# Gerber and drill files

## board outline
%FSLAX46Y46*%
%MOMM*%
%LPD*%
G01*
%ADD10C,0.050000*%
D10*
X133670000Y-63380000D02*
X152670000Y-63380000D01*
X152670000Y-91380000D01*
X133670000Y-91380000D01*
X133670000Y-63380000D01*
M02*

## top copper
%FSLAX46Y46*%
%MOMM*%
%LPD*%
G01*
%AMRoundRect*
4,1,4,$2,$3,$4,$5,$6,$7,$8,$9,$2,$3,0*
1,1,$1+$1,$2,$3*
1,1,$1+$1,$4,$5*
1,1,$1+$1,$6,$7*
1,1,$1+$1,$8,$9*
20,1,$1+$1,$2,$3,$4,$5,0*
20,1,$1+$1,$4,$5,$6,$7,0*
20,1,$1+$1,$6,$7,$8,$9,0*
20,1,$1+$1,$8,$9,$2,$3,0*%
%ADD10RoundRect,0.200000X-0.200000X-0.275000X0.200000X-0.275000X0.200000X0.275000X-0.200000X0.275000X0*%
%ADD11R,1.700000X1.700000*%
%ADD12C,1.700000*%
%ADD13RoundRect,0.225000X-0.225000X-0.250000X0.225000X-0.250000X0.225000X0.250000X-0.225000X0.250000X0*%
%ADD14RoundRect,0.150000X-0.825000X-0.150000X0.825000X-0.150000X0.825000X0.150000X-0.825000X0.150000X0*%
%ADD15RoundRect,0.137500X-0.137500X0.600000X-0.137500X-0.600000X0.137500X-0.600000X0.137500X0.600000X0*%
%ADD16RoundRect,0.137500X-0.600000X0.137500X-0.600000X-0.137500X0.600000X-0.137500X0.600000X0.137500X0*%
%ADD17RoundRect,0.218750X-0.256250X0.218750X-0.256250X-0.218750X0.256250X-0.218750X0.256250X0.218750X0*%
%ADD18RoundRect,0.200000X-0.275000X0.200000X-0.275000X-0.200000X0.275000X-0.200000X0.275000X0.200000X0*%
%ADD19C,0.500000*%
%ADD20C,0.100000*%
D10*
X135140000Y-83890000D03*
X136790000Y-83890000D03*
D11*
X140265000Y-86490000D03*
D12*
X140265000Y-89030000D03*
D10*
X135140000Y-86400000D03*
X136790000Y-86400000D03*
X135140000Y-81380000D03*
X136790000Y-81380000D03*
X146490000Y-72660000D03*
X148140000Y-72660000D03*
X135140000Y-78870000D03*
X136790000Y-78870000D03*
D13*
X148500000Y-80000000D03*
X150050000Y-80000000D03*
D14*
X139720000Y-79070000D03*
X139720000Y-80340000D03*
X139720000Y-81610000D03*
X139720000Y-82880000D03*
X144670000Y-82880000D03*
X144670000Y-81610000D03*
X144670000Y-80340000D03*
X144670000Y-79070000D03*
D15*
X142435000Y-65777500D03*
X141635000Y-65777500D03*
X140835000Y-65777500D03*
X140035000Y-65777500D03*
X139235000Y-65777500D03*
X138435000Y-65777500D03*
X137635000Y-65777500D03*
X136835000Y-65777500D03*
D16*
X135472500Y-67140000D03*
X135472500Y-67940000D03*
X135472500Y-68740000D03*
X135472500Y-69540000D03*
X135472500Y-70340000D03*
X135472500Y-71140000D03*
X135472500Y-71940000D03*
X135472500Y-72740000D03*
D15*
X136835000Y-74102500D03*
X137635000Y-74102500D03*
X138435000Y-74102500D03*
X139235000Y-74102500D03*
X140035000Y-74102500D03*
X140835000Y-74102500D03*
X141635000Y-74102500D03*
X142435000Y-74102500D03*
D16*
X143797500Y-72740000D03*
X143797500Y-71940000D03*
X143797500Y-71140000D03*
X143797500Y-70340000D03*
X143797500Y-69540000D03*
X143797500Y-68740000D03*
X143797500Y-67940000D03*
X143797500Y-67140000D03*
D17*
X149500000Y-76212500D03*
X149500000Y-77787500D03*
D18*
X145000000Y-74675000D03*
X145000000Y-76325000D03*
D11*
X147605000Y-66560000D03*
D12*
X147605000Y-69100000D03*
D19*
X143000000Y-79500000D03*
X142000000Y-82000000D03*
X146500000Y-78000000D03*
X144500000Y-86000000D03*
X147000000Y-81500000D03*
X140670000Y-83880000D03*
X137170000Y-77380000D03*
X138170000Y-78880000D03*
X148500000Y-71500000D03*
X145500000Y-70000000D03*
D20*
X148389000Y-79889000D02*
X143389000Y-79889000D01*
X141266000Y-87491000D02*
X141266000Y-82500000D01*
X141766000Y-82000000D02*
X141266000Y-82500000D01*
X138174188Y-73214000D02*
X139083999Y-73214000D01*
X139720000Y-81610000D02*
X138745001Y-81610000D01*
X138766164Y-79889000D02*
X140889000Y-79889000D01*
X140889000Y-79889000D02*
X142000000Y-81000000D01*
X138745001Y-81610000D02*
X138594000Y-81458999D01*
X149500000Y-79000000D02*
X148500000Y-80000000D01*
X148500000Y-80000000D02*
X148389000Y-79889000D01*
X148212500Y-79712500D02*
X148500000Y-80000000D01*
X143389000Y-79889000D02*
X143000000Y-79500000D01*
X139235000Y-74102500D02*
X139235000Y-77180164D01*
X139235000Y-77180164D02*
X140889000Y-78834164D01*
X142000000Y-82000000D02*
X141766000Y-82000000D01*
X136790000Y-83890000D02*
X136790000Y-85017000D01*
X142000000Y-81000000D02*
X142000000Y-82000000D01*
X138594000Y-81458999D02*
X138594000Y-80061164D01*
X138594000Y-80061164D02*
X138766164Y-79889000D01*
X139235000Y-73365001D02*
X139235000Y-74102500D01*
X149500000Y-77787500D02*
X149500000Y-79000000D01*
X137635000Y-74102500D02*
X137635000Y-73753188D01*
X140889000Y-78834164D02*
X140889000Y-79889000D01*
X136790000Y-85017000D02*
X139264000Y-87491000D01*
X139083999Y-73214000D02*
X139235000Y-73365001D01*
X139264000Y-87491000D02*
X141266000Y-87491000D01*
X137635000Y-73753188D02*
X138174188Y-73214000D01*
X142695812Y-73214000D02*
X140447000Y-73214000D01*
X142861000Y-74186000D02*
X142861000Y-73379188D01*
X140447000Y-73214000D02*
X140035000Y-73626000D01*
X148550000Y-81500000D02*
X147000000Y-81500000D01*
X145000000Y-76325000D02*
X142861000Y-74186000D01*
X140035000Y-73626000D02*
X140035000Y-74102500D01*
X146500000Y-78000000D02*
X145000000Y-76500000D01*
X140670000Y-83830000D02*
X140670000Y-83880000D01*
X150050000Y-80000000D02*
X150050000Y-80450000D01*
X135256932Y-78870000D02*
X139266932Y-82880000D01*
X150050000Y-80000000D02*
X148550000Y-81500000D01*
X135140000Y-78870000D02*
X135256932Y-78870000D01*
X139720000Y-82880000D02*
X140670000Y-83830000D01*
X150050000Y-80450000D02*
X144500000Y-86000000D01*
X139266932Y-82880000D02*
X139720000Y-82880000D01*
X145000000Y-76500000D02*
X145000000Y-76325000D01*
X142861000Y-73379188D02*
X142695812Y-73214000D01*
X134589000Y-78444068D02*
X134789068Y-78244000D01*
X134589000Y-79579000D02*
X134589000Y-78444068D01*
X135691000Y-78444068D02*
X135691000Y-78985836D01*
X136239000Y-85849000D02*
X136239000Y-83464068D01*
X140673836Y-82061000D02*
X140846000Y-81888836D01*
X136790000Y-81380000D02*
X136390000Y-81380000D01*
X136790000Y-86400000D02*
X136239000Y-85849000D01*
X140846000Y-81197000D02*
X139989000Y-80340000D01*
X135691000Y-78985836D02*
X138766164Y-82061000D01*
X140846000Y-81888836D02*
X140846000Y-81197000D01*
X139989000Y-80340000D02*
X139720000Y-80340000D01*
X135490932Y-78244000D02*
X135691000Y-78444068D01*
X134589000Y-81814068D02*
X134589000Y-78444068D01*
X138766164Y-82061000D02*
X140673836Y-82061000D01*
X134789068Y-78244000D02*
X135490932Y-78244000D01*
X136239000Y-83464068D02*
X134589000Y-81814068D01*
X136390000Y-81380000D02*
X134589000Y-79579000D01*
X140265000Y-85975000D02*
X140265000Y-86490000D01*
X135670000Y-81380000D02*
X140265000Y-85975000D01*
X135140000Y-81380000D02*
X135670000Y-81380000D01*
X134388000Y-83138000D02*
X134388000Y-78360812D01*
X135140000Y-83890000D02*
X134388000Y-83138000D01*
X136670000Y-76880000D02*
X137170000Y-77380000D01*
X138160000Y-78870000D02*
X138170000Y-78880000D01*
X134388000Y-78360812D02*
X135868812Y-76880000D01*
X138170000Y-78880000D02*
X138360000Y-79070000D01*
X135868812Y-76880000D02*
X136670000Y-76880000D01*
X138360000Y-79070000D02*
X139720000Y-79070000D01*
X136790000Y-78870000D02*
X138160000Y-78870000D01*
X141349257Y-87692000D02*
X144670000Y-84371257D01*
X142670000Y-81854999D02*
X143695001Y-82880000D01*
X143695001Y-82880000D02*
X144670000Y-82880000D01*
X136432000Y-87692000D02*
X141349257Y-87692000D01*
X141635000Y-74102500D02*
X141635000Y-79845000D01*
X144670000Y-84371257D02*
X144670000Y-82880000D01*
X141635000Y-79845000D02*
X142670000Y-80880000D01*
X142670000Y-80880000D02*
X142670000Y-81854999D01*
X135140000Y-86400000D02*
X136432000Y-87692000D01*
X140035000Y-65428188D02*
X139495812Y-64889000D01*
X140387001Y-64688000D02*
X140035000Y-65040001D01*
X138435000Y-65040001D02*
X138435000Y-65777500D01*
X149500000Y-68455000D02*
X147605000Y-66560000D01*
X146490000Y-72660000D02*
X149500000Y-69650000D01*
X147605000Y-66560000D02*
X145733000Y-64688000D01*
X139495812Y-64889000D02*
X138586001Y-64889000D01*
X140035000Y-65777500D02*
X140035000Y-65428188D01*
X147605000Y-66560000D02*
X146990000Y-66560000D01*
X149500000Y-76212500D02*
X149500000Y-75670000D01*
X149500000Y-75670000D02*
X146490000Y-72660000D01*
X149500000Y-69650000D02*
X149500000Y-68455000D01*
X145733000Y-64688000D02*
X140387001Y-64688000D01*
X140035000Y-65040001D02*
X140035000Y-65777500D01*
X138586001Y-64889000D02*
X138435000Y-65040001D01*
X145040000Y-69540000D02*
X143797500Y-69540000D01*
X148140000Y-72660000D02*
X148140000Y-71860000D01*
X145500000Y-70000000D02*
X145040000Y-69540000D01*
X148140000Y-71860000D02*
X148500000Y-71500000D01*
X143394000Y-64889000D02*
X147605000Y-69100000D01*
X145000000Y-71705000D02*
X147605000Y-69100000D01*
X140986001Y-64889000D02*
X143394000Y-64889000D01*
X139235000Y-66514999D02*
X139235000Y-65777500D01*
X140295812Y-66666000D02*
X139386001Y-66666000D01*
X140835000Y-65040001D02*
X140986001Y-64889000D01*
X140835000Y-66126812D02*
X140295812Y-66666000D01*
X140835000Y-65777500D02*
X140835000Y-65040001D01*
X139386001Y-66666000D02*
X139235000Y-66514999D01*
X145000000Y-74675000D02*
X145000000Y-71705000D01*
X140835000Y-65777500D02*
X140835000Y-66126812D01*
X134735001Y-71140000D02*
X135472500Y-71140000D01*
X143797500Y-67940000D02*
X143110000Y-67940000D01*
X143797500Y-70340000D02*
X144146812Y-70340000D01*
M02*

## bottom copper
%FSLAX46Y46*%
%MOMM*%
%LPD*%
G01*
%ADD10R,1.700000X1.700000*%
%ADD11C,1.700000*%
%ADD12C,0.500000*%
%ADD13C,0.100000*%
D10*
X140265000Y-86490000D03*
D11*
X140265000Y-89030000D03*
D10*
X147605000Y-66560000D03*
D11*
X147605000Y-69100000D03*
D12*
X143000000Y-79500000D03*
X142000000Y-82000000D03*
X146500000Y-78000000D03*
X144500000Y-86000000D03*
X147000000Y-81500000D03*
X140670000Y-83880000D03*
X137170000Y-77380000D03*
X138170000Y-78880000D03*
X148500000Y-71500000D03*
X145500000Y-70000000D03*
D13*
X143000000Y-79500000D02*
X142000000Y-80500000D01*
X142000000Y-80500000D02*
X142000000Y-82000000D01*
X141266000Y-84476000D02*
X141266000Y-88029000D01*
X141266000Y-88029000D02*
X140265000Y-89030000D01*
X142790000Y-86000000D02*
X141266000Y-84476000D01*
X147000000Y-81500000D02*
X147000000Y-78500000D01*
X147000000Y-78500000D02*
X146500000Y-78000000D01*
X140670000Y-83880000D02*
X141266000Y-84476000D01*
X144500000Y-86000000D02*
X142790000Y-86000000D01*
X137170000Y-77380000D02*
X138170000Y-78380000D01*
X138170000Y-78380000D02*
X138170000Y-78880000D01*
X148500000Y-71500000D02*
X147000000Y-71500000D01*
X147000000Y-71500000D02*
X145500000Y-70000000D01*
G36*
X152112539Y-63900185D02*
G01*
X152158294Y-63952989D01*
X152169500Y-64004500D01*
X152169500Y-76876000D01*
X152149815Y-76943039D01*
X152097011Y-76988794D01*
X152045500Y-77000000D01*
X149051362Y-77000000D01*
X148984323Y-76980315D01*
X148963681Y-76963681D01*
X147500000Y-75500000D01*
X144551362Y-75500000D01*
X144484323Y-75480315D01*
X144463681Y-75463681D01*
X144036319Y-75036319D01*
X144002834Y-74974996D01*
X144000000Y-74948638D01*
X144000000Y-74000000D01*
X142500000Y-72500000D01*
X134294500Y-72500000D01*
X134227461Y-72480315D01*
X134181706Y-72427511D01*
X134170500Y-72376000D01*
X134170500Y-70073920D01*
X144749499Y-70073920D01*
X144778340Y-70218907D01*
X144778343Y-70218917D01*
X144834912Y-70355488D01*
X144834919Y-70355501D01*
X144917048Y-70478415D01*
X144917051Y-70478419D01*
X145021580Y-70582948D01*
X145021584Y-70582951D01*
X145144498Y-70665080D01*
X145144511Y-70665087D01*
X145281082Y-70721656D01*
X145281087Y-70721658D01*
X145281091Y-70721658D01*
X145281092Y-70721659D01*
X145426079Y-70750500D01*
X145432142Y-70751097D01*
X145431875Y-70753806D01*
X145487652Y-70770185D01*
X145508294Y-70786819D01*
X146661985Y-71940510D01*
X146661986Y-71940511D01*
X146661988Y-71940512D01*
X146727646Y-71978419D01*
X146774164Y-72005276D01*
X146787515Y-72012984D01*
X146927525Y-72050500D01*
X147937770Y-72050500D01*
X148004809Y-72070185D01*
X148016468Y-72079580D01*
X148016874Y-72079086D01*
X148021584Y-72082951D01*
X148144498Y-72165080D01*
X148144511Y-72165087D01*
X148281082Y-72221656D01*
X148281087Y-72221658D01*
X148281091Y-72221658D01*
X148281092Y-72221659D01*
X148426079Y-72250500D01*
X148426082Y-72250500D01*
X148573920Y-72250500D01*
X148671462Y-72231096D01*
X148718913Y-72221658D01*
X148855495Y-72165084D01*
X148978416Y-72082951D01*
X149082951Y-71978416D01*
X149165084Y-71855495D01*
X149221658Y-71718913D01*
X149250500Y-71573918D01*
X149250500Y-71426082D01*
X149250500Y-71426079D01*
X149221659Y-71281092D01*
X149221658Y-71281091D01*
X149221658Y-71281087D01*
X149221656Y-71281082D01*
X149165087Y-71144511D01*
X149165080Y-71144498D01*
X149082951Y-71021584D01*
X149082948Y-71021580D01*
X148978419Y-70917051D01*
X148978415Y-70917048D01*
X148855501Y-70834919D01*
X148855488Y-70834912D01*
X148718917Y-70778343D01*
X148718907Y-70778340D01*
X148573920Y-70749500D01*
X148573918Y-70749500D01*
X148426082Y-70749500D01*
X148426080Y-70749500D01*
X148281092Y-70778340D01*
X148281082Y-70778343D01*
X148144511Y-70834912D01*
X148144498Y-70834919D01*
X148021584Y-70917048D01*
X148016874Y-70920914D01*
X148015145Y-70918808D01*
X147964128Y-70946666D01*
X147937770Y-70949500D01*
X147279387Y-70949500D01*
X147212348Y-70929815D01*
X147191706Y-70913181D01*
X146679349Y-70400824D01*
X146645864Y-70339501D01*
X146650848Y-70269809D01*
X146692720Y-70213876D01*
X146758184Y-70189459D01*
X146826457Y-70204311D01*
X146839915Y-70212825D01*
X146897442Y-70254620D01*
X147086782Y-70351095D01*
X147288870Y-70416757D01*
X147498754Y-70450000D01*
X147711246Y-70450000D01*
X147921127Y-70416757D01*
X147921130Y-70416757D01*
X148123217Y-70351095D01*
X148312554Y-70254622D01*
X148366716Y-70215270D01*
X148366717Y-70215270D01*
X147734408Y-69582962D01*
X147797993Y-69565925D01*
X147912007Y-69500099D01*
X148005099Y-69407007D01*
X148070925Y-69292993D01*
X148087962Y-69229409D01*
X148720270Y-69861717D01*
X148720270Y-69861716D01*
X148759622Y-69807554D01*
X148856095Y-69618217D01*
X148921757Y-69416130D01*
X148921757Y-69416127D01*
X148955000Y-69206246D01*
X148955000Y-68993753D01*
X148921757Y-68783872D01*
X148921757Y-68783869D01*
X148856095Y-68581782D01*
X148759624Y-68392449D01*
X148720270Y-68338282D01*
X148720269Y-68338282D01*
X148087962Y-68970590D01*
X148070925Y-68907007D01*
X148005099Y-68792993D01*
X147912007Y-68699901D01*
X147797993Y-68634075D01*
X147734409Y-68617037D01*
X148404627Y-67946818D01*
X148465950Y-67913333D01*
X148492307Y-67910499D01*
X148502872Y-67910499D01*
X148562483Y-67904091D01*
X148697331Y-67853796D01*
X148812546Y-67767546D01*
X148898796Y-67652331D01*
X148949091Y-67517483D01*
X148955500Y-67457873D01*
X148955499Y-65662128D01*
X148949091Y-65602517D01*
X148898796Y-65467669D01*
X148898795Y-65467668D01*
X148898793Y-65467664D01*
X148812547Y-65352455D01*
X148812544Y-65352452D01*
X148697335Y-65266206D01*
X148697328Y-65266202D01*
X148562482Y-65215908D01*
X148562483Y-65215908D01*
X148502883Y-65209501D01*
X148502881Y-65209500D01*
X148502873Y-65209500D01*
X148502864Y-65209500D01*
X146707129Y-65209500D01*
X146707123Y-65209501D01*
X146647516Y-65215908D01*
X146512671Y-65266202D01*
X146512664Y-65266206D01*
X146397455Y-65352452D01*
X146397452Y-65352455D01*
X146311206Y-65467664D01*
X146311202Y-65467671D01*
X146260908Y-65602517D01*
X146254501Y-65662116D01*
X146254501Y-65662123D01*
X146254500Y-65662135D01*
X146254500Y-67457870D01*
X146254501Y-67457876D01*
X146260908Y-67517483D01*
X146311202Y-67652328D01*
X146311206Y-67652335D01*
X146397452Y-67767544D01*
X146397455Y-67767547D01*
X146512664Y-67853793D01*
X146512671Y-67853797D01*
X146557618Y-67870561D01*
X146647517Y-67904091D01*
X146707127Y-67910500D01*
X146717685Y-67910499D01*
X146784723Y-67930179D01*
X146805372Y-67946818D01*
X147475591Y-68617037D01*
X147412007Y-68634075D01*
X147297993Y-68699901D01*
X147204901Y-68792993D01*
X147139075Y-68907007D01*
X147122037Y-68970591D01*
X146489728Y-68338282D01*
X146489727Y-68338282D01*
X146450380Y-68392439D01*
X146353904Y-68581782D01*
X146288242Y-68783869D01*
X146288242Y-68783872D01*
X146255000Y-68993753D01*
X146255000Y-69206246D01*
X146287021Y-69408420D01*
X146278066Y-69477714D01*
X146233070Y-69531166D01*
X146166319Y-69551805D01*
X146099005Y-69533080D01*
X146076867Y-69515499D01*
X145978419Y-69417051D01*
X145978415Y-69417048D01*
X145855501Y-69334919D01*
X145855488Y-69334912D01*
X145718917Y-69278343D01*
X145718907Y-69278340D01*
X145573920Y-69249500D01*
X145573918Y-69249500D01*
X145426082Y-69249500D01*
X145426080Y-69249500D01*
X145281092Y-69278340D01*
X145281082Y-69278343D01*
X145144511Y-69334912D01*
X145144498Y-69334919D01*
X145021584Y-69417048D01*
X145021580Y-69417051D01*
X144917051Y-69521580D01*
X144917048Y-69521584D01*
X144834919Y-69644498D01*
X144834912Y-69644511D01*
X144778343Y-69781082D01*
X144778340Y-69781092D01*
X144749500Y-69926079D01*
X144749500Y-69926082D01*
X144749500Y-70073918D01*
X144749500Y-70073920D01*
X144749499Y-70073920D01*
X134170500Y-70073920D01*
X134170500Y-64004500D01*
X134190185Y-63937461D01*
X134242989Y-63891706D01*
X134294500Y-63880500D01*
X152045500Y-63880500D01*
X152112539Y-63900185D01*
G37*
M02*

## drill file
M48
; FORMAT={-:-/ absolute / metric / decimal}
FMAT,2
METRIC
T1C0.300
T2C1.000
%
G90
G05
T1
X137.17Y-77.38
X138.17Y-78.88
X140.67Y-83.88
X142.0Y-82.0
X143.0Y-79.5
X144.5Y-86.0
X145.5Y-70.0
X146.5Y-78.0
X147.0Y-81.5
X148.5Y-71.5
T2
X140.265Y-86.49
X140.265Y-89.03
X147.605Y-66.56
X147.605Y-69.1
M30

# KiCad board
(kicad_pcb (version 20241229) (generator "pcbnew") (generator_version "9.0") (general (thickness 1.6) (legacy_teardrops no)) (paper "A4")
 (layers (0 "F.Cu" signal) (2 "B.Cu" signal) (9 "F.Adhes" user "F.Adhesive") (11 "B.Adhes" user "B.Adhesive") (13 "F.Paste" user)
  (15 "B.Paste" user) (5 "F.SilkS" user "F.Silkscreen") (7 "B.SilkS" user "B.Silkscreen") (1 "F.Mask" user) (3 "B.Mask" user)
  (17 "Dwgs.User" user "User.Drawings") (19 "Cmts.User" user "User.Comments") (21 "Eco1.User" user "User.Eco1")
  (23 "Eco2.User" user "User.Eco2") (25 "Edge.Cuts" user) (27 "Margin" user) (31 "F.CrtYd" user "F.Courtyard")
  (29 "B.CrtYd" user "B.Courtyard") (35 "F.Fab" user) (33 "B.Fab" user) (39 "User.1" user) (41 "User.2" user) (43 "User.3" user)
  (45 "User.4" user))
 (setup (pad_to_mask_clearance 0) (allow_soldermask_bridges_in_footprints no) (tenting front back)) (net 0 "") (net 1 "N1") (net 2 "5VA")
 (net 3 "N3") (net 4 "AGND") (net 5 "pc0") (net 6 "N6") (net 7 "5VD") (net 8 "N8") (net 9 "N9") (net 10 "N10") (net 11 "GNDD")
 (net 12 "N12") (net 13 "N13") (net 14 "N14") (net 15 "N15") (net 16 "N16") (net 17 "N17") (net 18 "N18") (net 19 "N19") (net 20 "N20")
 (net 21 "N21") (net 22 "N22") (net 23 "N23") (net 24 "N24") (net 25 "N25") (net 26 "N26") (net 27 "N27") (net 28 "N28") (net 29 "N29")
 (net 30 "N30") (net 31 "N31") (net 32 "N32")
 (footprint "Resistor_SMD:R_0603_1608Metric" (layer "F.Cu") (at 135.965 83.89)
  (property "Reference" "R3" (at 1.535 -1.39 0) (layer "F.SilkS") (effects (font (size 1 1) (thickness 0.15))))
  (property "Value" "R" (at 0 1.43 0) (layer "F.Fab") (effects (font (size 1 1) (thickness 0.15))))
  (pad "1" smd roundrect (at -0.825 0) (size 0.8 0.95) (layers "F.Cu" "F.Mask" "F.Paste") (roundrect_rratio 0.25) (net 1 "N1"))
  (pad "2" smd roundrect (at 0.825 0) (size 0.8 0.95) (layers "F.Cu" "F.Mask" "F.Paste") (roundrect_rratio 0.25) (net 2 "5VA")))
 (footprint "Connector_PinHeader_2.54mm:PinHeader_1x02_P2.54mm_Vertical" (layer "F.Cu") (at 140.265 86.49)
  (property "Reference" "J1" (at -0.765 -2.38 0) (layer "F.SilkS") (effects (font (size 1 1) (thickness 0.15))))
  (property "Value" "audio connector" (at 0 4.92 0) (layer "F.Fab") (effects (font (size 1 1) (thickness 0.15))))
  (pad "1" thru_hole rect (at 0 0) (size 1.7 1.7) (drill 1) (layers "*.Cu" "*.Mask") (remove_unused_layers no) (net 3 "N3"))
  (pad "2" thru_hole circle (at 0 2.54) (size 1.7 1.7) (drill 1) (layers "*.Cu" "*.Mask") (remove_unused_layers no) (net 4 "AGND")))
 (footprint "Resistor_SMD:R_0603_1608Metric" (layer "F.Cu") (at 135.965 86.4)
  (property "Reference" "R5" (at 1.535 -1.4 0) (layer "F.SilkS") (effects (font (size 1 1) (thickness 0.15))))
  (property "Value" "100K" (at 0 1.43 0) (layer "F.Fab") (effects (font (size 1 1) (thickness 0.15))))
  (pad "1" smd roundrect (at -0.825 0) (size 0.8 0.95) (layers "F.Cu" "F.Mask" "F.Paste") (roundrect_rratio 0.25) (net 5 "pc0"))
  (pad "2" smd roundrect (at 0.825 0) (size 0.8 0.95) (layers "F.Cu" "F.Mask" "F.Paste") (roundrect_rratio 0.25) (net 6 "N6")))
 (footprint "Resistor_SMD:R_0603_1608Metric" (layer "F.Cu") (at 135.965 81.38)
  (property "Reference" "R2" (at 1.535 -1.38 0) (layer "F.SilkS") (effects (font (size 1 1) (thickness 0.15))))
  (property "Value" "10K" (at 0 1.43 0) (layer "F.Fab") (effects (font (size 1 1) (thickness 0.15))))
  (pad "1" smd roundrect (at -0.825 0) (size 0.8 0.95) (layers "F.Cu" "F.Mask" "F.Paste") (roundrect_rratio 0.25) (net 3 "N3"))
  (pad "2" smd roundrect (at 0.825 0) (size 0.8 0.95) (layers "F.Cu" "F.Mask" "F.Paste") (roundrect_rratio 0.25) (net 6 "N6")))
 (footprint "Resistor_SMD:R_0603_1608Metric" (layer "F.Cu") (at 147.315 72.66)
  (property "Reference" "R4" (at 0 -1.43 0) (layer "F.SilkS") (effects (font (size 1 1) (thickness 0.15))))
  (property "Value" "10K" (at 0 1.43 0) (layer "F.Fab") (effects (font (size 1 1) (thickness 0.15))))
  (pad "1" smd roundrect (at -0.825 0) (size 0.8 0.95) (layers "F.Cu" "F.Mask" "F.Paste") (roundrect_rratio 0.25) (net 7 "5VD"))
  (pad "2" smd roundrect (at 0.825 0) (size 0.8 0.95) (layers "F.Cu" "F.Mask" "F.Paste") (roundrect_rratio 0.25) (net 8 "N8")))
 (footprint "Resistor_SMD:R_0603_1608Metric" (layer "F.Cu") (at 135.965 78.87)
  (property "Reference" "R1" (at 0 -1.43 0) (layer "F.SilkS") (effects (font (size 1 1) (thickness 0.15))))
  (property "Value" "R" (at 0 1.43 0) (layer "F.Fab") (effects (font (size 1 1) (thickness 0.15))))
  (pad "1" smd roundrect (at -0.825 0) (size 0.8 0.95) (layers "F.Cu" "F.Mask" "F.Paste") (roundrect_rratio 0.25) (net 4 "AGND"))
  (pad "2" smd roundrect (at 0.825 0) (size 0.8 0.95) (layers "F.Cu" "F.Mask" "F.Paste") (roundrect_rratio 0.25) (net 1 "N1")))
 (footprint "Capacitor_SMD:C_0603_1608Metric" (layer "F.Cu") (at 149.275 80)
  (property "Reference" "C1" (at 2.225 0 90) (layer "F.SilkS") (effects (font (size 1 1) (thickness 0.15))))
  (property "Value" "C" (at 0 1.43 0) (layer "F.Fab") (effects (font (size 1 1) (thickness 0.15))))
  (pad "1" smd roundrect (at -0.775 0) (size 0.9 0.95) (layers "F.Cu" "F.Mask" "F.Paste") (roundrect_rratio 0.25) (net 2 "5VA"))
  (pad "2" smd roundrect (at 0.775 0) (size 0.9 0.95) (layers "F.Cu" "F.Mask" "F.Paste") (roundrect_rratio 0.25) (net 4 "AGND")))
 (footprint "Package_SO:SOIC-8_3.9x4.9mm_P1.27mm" (layer "F.Cu") (at 142.195 80.975)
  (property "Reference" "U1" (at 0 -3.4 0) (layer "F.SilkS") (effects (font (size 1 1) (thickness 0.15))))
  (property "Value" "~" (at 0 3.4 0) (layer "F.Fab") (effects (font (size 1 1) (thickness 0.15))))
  (pad "1" smd roundrect (at -2.475 -1.905) (size 1.95 0.6) (layers "F.Cu" "F.Mask" "F.Paste") (roundrect_rratio 0.25) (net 1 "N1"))
  (pad "2" smd roundrect (at -2.475 -0.635) (size 1.95 0.6) (layers "F.Cu" "F.Mask" "F.Paste") (roundrect_rratio 0.25) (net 6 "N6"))
  (pad "3" smd roundrect (at -2.475 0.635) (size 1.95 0.6) (layers "F.Cu" "F.Mask" "F.Paste") (roundrect_rratio 0.25) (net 2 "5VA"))
  (pad "4" smd roundrect (at -2.475 1.905) (size 1.95 0.6) (layers "F.Cu" "F.Mask" "F.Paste") (roundrect_rratio 0.25) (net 4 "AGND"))
  (pad "5" smd roundrect (at 2.475 1.905) (size 1.95 0.6) (layers "F.Cu" "F.Mask" "F.Paste") (roundrect_rratio 0.25) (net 5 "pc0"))
  (pad "6" smd roundrect (at 2.475 0.635) (size 1.95 0.6) (layers "F.Cu" "F.Mask" "F.Paste") (roundrect_rratio 0.25))
  (pad "7" smd roundrect (at 2.475 -0.635) (size 1.95 0.6) (layers "F.Cu" "F.Mask" "F.Paste") (roundrect_rratio 0.25))
  (pad "8" smd roundrect (at 2.475 -1.905) (size 1.95 0.6) (layers "F.Cu" "F.Mask" "F.Paste") (roundrect_rratio 0.25)))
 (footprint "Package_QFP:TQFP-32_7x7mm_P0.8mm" (layer "F.Cu") (at 139.635 69.94 -90)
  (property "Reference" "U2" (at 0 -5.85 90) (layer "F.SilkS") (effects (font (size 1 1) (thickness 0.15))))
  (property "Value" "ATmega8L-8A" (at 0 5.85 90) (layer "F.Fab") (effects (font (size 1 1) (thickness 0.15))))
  (pad "1" smd roundrect (at -4.1625 -2.8 270) (size 1.475 0.55) (layers "F.Cu" "F.Mask" "F.Paste") (roundrect_rratio 0.25) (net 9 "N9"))
  (pad "2" smd roundrect (at -4.1625 -2 270) (size 1.475 0.55) (layers "F.Cu" "F.Mask" "F.Paste") (roundrect_rratio 0.25) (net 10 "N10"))
  (pad "3" smd roundrect (at -4.1625 -1.2 270) (size 1.475 0.55) (layers "F.Cu" "F.Mask" "F.Paste") (roundrect_rratio 0.25) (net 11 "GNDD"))
  (pad "4" smd roundrect (at -4.1625 -0.4 270) (size 1.475 0.55) (layers "F.Cu" "F.Mask" "F.Paste") (roundrect_rratio 0.25) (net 7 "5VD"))
  (pad "5" smd roundrect (at -4.1625 0.4 270) (size 1.475 0.55) (layers "F.Cu" "F.Mask" "F.Paste") (roundrect_rratio 0.25) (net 11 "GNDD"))
  (pad "6" smd roundrect (at -4.1625 1.2 270) (size 1.475 0.55) (layers "F.Cu" "F.Mask" "F.Paste") (roundrect_rratio 0.25) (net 7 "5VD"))
  (pad "7" smd roundrect (at -4.1625 2 270) (size 1.475 0.55) (layers "F.Cu" "F.Mask" "F.Paste") (roundrect_rratio 0.25) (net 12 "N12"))
  (pad "8" smd roundrect (at -4.1625 2.8 270) (size 1.475 0.55) (layers "F.Cu" "F.Mask" "F.Paste") (roundrect_rratio 0.25) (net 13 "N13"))
  (pad "9" smd roundrect (at -2.8 4.1625 270) (size 0.55 1.475) (layers "F.Cu" "F.Mask" "F.Paste") (roundrect_rratio 0.25) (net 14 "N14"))
  (pad "10" smd roundrect (at -2 4.1625 270) (size 0.55 1.475) (layers "F.Cu" "F.Mask" "F.Paste") (roundrect_rratio 0.25) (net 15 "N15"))
  (pad "11" smd roundrect (at -1.2 4.1625 270) (size 0.55 1.475) (layers "F.Cu" "F.Mask" "F.Paste") (roundrect_rratio 0.25) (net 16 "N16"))
  (pad "12" smd roundrect (at -0.4 4.1625 270) (size 0.55 1.475) (layers "F.Cu" "F.Mask" "F.Paste") (roundrect_rratio 0.25) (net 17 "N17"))
  (pad "13" smd roundrect (at 0.4 4.1625 270) (size 0.55 1.475) (layers "F.Cu" "F.Mask" "F.Paste") (roundrect_rratio 0.25) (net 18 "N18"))
  (pad "14" smd roundrect (at 1.2 4.1625 270) (size 0.55 1.475) (layers "F.Cu" "F.Mask" "F.Paste") (roundrect_rratio 0.25) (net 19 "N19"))
  (pad "15" smd roundrect (at 2 4.1625 270) (size 0.55 1.475) (layers "F.Cu" "F.Mask" "F.Paste") (roundrect_rratio 0.25) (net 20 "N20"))
  (pad "16" smd roundrect (at 2.8 4.1625 270) (size 0.55 1.475) (layers "F.Cu" "F.Mask" "F.Paste") (roundrect_rratio 0.25) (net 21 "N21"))
  (pad "17" smd roundrect (at 4.1625 2.8 270) (size 1.475 0.55) (layers "F.Cu" "F.Mask" "F.Paste") (roundrect_rratio 0.25) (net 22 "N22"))
  (pad "18" smd roundrect (at 4.1625 2 270) (size 1.475 0.55) (layers "F.Cu" "F.Mask" "F.Paste") (roundrect_rratio 0.25) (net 2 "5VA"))
  (pad "19" smd roundrect (at 4.1625 1.2 270) (size 1.475 0.55) (layers "F.Cu" "F.Mask" "F.Paste") (roundrect_rratio 0.25) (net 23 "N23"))
  (pad "20" smd roundrect (at 4.1625 0.4 270) (size 1.475 0.55) (layers "F.Cu" "F.Mask" "F.Paste") (roundrect_rratio 0.25) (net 2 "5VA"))
  (pad "21" smd roundrect (at 4.1625 -0.4 270) (size 1.475 0.55) (layers "F.Cu" "F.Mask" "F.Paste") (roundrect_rratio 0.25) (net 4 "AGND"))
  (pad "22" smd roundrect (at 4.1625 -1.2 270) (size 1.475 0.55) (layers "F.Cu" "F.Mask" "F.Paste") (roundrect_rratio 0.25) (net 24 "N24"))
  (pad "23" smd roundrect (at 4.1625 -2 270) (size 1.475 0.55) (layers "F.Cu" "F.Mask" "F.Paste") (roundrect_rratio 0.25) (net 5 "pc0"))
  (pad "24" smd roundrect (at 4.1625 -2.8 270) (size 1.475 0.55) (layers "F.Cu" "F.Mask" "F.Paste") (roundrect_rratio 0.25) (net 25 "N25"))
  (pad "25" smd roundrect (at 2.8 -4.1625 270) (size 0.55 1.475) (layers "F.Cu" "F.Mask" "F.Paste") (roundrect_rratio 0.25) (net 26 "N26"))
  (pad "26" smd roundrect (at 2 -4.1625 270) (size 0.55 1.475) (layers "F.Cu" "F.Mask" "F.Paste") (roundrect_rratio 0.25) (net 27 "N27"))
  (pad "27" smd roundrect (at 1.2 -4.1625 270) (size 0.55 1.475) (layers "F.Cu" "F.Mask" "F.Paste") (roundrect_rratio 0.25) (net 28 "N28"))
  (pad "28" smd roundrect (at 0.4 -4.1625 270) (size 0.55 1.475) (layers "F.Cu" "F.Mask" "F.Paste") (roundrect_rratio 0.25) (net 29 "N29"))
  (pad "29" smd roundrect (at -0.4 -4.1625 270) (size 0.55 1.475) (layers "F.Cu" "F.Mask" "F.Paste") (roundrect_rratio 0.25) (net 8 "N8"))
  (pad "30" smd roundrect (at -1.2 -4.1625 270) (size 0.55 1.475) (layers "F.Cu" "F.Mask" "F.Paste") (roundrect_rratio 0.25) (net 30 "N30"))
  (pad "31" smd roundrect (at -2 -4.1625 270) (size 0.55 1.475) (layers "F.Cu" "F.Mask" "F.Paste") (roundrect_rratio 0.25) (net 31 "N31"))
  (pad "32" smd roundrect (at -2.8 -4.1625 270) (size 0.55 1.475) (layers "F.Cu" "F.Mask" "F.Paste") (roundrect_rratio 0.25) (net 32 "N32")))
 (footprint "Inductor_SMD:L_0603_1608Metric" (layer "F.Cu") (at 149.5 77 -90)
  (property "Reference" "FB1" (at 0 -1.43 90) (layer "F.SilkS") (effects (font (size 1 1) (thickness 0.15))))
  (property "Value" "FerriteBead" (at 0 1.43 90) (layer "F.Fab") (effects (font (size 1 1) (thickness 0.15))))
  (pad "1" smd roundrect (at -0.7875 0 270) (size 0.875 0.95) (layers "F.Cu" "F.Mask" "F.Paste") (roundrect_rratio 0.25) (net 7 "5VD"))
  (pad "2" smd roundrect (at 0.7875 0 270) (size 0.875 0.95) (layers "F.Cu" "F.Mask" "F.Paste") (roundrect_rratio 0.25) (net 2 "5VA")))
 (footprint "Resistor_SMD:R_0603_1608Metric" (layer "F.Cu") (at 145 75.5 -90)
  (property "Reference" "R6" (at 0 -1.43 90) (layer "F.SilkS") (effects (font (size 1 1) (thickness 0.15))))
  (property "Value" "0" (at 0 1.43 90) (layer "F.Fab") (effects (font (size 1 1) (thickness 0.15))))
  (pad "1" smd roundrect (at -0.825 0 270) (size 0.8 0.95) (layers "F.Cu" "F.Mask" "F.Paste") (roundrect_rratio 0.25) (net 11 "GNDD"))
  (pad "2" smd roundrect (at 0.825 0 270) (size 0.8 0.95) (layers "F.Cu" "F.Mask" "F.Paste") (roundrect_rratio 0.25) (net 4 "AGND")))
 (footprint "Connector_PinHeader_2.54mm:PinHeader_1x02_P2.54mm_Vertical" (layer "F.Cu") (at 147.605 66.56)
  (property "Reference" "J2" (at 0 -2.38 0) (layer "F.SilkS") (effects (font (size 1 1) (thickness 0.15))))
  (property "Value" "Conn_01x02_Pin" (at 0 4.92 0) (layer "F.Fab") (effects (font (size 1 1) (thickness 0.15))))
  (pad "1" thru_hole rect (at 0 0) (size 1.7 1.7) (drill 1) (layers "*.Cu" "*.Mask") (remove_unused_layers no) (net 7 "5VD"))
  (pad "2" thru_hole circle (at 0 2.54) (size 1.7 1.7) (drill 1) (layers "*.Cu" "*.Mask") (remove_unused_layers no) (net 11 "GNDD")))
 (gr_rect (start 133.67 63.38) (end 152.67 91.38) (stroke (width 0.05) (type default)) (fill no) (layer "Edge.Cuts"))
 (segment (start 148.389 79.889) (end 143.389 79.889) (width 0.1) (layer "F.Cu") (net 2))
 (segment (start 141.266 87.491) (end 141.266 82.5) (width 0.1) (layer "F.Cu") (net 2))
 (segment (start 141.766 82) (end 141.266 82.5) (width 0.1) (layer "F.Cu") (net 2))
 (segment (start 138.174188 73.214) (end 139.083999 73.214) (width 0.1) (layer "F.Cu") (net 2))
 (segment (start 139.72 81.61) (end 138.745001 81.61) (width 0.1) (layer "F.Cu") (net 2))
 (segment (start 138.766164 79.889) (end 140.889 79.889) (width 0.1) (layer "F.Cu") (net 2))
 (segment (start 140.889 79.889) (end 142 81) (width 0.1) (layer "F.Cu") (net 2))
 (segment (start 138.745001 81.61) (end 138.594 81.458999) (width 0.1) (layer "F.Cu") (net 2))
 (segment (start 149.5 79) (end 148.5 80) (width 0.1) (layer "F.Cu") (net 2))
 (segment (start 148.5 80) (end 148.389 79.889) (width 0.1) (layer "F.Cu") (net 2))
 (segment (start 148.2125 79.7125) (end 148.5 80) (width 0.1) (layer "F.Cu") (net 2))
 (segment (start 143.389 79.889) (end 143 79.5) (width 0.1) (layer "F.Cu") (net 2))
 (segment (start 139.235 74.1025) (end 139.235 77.180164) (width 0.1) (layer "F.Cu") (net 2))
 (segment (start 139.235 77.180164) (end 140.889 78.834164) (width 0.1) (layer "F.Cu") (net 2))
 (segment (start 142 82) (end 141.766 82) (width 0.1) (layer "F.Cu") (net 2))
 (segment (start 136.79 83.89) (end 136.79 85.017) (width 0.1) (layer "F.Cu") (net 2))
 (segment (start 142 81) (end 142 82) (width 0.1) (layer "F.Cu") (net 2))
 (segment (start 138.594 81.458999) (end 138.594 80.061164) (width 0.1) (layer "F.Cu") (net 2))
 (segment (start 138.594 80.061164) (end 138.766164 79.889) (width 0.1) (layer "F.Cu") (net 2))
 (segment (start 139.235 73.365001) (end 139.235 74.1025) (width 0.1) (layer "F.Cu") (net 2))
 (segment (start 149.5 77.7875) (end 149.5 79) (width 0.1) (layer "F.Cu") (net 2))
 (segment (start 137.635 74.1025) (end 137.635 73.753188) (width 0.1) (layer "F.Cu") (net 2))
 (segment (start 140.889 78.834164) (end 140.889 79.889) (width 0.1) (layer "F.Cu") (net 2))
 (segment (start 136.79 85.017) (end 139.264 87.491) (width 0.1) (layer "F.Cu") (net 2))
 (segment (start 139.083999 73.214) (end 139.235 73.365001) (width 0.1) (layer "F.Cu") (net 2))
 (segment (start 139.264 87.491) (end 141.266 87.491) (width 0.1) (layer "F.Cu") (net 2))
 (segment (start 137.635 73.753188) (end 138.174188 73.214) (width 0.1) (layer "F.Cu") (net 2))
 (via (at 143 79.5) (size 0.5) (drill 0.3) (layers "F.Cu" "B.Cu") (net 2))
 (via (at 142 82) (size 0.5) (drill 0.3) (layers "F.Cu" "B.Cu") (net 2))
 (segment (start 143 79.5) (end 142 80.5) (width 0.1) (layer "B.Cu") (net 2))
 (segment (start 142 80.5) (end 142 82) (width 0.1) (layer "B.Cu") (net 2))
 (segment (start 142.695812 73.214) (end 140.447 73.214) (width 0.1) (layer "F.Cu") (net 4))
 (segment (start 142.861 74.186) (end 142.861 73.379188) (width 0.1) (layer "F.Cu") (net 4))
 (segment (start 140.447 73.214) (end 140.035 73.626) (width 0.1) (layer "F.Cu") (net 4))
 (segment (start 148.55 81.5) (end 147 81.5) (width 0.1) (layer "F.Cu") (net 4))
 (segment (start 145 76.325) (end 142.861 74.186) (width 0.1) (layer "F.Cu") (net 4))
 (segment (start 140.035 73.626) (end 140.035 74.1025) (width 0.1) (layer "F.Cu") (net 4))
 (segment (start 146.5 78) (end 145 76.5) (width 0.1) (layer "F.Cu") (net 4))
 (segment (start 140.67 83.83) (end 140.67 83.88) (width 0.1) (layer "F.Cu") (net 4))
 (segment (start 150.05 80) (end 150.05 80.45) (width 0.1) (layer "F.Cu") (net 4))
 (segment (start 135.256932 78.87) (end 139.266932 82.88) (width 0.1) (layer "F.Cu") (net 4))
 (segment (start 150.05 80) (end 148.55 81.5) (width 0.1) (layer "F.Cu") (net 4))
 (segment (start 135.14 78.87) (end 135.256932 78.87) (width 0.1) (layer "F.Cu") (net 4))
 (segment (start 139.72 82.88) (end 140.67 83.83) (width 0.1) (layer "F.Cu") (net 4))
 (segment (start 150.05 80.45) (end 144.5 86) (width 0.1) (layer "F.Cu") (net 4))
 (segment (start 139.266932 82.88) (end 139.72 82.88) (width 0.1) (layer "F.Cu") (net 4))
 (segment (start 145 76.5) (end 145 76.325) (width 0.1) (layer "F.Cu") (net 4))
 (segment (start 142.861 73.379188) (end 142.695812 73.214) (width 0.1) (layer "F.Cu") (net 4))
 (via (at 146.5 78) (size 0.5) (drill 0.3) (layers "F.Cu" "B.Cu") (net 4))
 (via (at 144.5 86) (size 0.5) (drill 0.3) (layers "F.Cu" "B.Cu") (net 4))
 (via (at 147 81.5) (size 0.5) (drill 0.3) (layers "F.Cu" "B.Cu") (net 4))
 (via (at 140.67 83.88) (size 0.5) (drill 0.3) (layers "F.Cu" "B.Cu") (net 4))
 (segment (start 141.266 84.476) (end 141.266 88.029) (width 0.1) (layer "B.Cu") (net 4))
 (segment (start 141.266 88.029) (end 140.265 89.03) (width 0.1) (layer "B.Cu") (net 4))
 (segment (start 142.79 86) (end 141.266 84.476) (width 0.1) (layer "B.Cu") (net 4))
 (segment (start 147 81.5) (end 147 78.5) (width 0.1) (layer "B.Cu") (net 4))
 (segment (start 147 78.5) (end 146.5 78) (width 0.1) (layer "B.Cu") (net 4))
 (segment (start 140.67 83.88) (end 141.266 84.476) (width 0.1) (layer "B.Cu") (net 4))
 (segment (start 144.5 86) (end 142.79 86) (width 0.1) (layer "B.Cu") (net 4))
 (segment (start 134.589 78.444068) (end 134.789068 78.244) (width 0.1) (layer "F.Cu") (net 6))
 (segment (start 134.589 79.579) (end 134.589 78.444068) (width 0.1) (layer "F.Cu") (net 6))
 (segment (start 135.691 78.444068) (end 135.691 78.985836) (width 0.1) (layer "F.Cu") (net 6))
 (segment (start 136.239 85.849) (end 136.239 83.464068) (width 0.1) (layer "F.Cu") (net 6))
 (segment (start 140.673836 82.061) (end 140.846 81.888836) (width 0.1) (layer "F.Cu") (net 6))
 (segment (start 136.79 81.38) (end 136.39 81.38) (width 0.1) (layer "F.Cu") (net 6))
 (segment (start 136.79 86.4) (end 136.239 85.849) (width 0.1) (layer "F.Cu") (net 6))
 (segment (start 140.846 81.197) (end 139.989 80.34) (width 0.1) (layer "F.Cu") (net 6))
 (segment (start 135.691 78.985836) (end 138.766164 82.061) (width 0.1) (layer "F.Cu") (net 6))
 (segment (start 140.846 81.888836) (end 140.846 81.197) (width 0.1) (layer "F.Cu") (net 6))
 (segment (start 139.989 80.34) (end 139.72 80.34) (width 0.1) (layer "F.Cu") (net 6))
 (segment (start 135.490932 78.244) (end 135.691 78.444068) (width 0.1) (layer "F.Cu") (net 6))
 (segment (start 134.589 81.814068) (end 134.589 78.444068) (width 0.1) (layer "F.Cu") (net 6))
 (segment (start 138.766164 82.061) (end 140.673836 82.061) (width 0.1) (layer "F.Cu") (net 6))
 (segment (start 134.789068 78.244) (end 135.490932 78.244) (width 0.1) (layer "F.Cu") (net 6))
 (segment (start 136.239 83.464068) (end 134.589 81.814068) (width 0.1) (layer "F.Cu") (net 6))
 (segment (start 136.39 81.38) (end 134.589 79.579) (width 0.1) (layer "F.Cu") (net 6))
 (segment (start 140.265 85.975) (end 140.265 86.49) (width 0.1) (layer "F.Cu") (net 3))
 (segment (start 135.67 81.38) (end 140.265 85.975) (width 0.1) (layer "F.Cu") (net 3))
 (segment (start 135.14 81.38) (end 135.67 81.38) (width 0.1) (layer "F.Cu") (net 3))
 (segment (start 134.388 83.138) (end 134.388 78.360812) (width 0.1) (layer "F.Cu") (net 1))
 (segment (start 135.14 83.89) (end 134.388 83.138) (width 0.1) (layer "F.Cu") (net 1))
 (segment (start 136.67 76.88) (end 137.17 77.38) (width 0.1) (layer "F.Cu") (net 1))
 (segment (start 138.16 78.87) (end 138.17 78.88) (width 0.1) (layer "F.Cu") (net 1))
 (segment (start 134.388 78.360812) (end 135.868812 76.88) (width 0.1) (layer "F.Cu") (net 1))
 (segment (start 138.17 78.88) (end 138.36 79.07) (width 0.1) (layer "F.Cu") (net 1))
 (segment (start 135.868812 76.88) (end 136.67 76.88) (width 0.1) (layer "F.Cu") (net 1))
 (segment (start 138.36 79.07) (end 139.72 79.07) (width 0.1) (layer "F.Cu") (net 1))
 (segment (start 136.79 78.87) (end 138.16 78.87) (width 0.1) (layer "F.Cu") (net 1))
 (via (at 137.17 77.38) (size 0.5) (drill 0.3) (layers "F.Cu" "B.Cu") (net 1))
 (via (at 138.17 78.88) (size 0.5) (drill 0.3) (layers "F.Cu" "B.Cu") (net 1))
 (segment (start 137.17 77.38) (end 138.17 78.38) (width 0.1) (layer "B.Cu") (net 1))
 (segment (start 138.17 78.38) (end 138.17 78.88) (width 0.1) (layer "B.Cu") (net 1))
 (segment (start 141.349257 87.692) (end 144.67 84.371257) (width 0.1) (layer "F.Cu") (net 5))
 (segment (start 142.67 81.854999) (end 143.695001 82.88) (width 0.1) (layer "F.Cu") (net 5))
 (segment (start 143.695001 82.88) (end 144.67 82.88) (width 0.1) (layer "F.Cu") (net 5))
 (segment (start 136.432 87.692) (end 141.349257 87.692) (width 0.1) (layer "F.Cu") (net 5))
 (segment (start 141.635 74.1025) (end 141.635 79.845) (width 0.1) (layer "F.Cu") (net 5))
 (segment (start 144.67 84.371257) (end 144.67 82.88) (width 0.1) (layer "F.Cu") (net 5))
 (segment (start 141.635 79.845) (end 142.67 80.88) (width 0.1) (layer "F.Cu") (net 5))
 (segment (start 142.67 80.88) (end 142.67 81.854999) (width 0.1) (layer "F.Cu") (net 5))
 (segment (start 135.14 86.4) (end 136.432 87.692) (width 0.1) (layer "F.Cu") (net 5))
 (segment (start 140.035 65.428188) (end 139.495812 64.889) (width 0.1) (layer "F.Cu") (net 7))
 (segment (start 140.387001 64.688) (end 140.035 65.040001) (width 0.1) (layer "F.Cu") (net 7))
 (segment (start 138.435 65.040001) (end 138.435 65.7775) (width 0.1) (layer "F.Cu") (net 7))
 (segment (start 149.5 68.455) (end 147.605 66.56) (width 0.1) (layer "F.Cu") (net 7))
 (segment (start 146.49 72.66) (end 149.5 69.65) (width 0.1) (layer "F.Cu") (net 7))
 (segment (start 147.605 66.56) (end 145.733 64.688) (width 0.1) (layer "F.Cu") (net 7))
 (segment (start 139.495812 64.889) (end 138.586001 64.889) (width 0.1) (layer "F.Cu") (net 7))
 (segment (start 140.035 65.7775) (end 140.035 65.428188) (width 0.1) (layer "F.Cu") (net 7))
 (segment (start 147.605 66.56) (end 146.99 66.56) (width 0.1) (layer "F.Cu") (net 7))
 (segment (start 149.5 76.2125) (end 149.5 75.67) (width 0.1) (layer "F.Cu") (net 7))
 (segment (start 149.5 75.67) (end 146.49 72.66) (width 0.1) (layer "F.Cu") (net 7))
 (segment (start 149.5 69.65) (end 149.5 68.455) (width 0.1) (layer "F.Cu") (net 7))
 (segment (start 145.733 64.688) (end 140.387001 64.688) (width 0.1) (layer "F.Cu") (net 7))
 (segment (start 140.035 65.040001) (end 140.035 65.7775) (width 0.1) (layer "F.Cu") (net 7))
 (segment (start 138.586001 64.889) (end 138.435 65.040001) (width 0.1) (layer "F.Cu") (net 7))
 (segment (start 145.04 69.54) (end 143.7975 69.54) (width 0.1) (layer "F.Cu") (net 8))
 (segment (start 148.14 72.66) (end 148.14 71.86) (width 0.1) (layer "F.Cu") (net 8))
 (segment (start 145.5 70) (end 145.04 69.54) (width 0.1) (layer "F.Cu") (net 8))
 (segment (start 148.14 71.86) (end 148.5 71.5) (width 0.1) (layer "F.Cu") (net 8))
 (via (at 148.5 71.5) (size 0.5) (drill 0.3) (layers "F.Cu" "B.Cu") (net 8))
 (via (at 145.5 70) (size 0.5) (drill 0.3) (layers "F.Cu" "B.Cu") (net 8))
 (segment (start 148.5 71.5) (end 147 71.5) (width 0.1) (layer "B.Cu") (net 8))
 (segment (start 147 71.5) (end 145.5 70) (width 0.1) (layer "B.Cu") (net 8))
 (segment (start 143.394 64.889) (end 147.605 69.1) (width 0.1) (layer "F.Cu") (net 11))
 (segment (start 145 71.705) (end 147.605 69.1) (width 0.1) (layer "F.Cu") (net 11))
 (segment (start 140.986001 64.889) (end 143.394 64.889) (width 0.1) (layer "F.Cu") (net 11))
 (segment (start 139.235 66.514999) (end 139.235 65.7775) (width 0.1) (layer "F.Cu") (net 11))
 (segment (start 140.295812 66.666) (end 139.386001 66.666) (width 0.1) (layer "F.Cu") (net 11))
 (segment (start 140.835 65.040001) (end 140.986001 64.889) (width 0.1) (layer "F.Cu") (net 11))
 (segment (start 140.835 66.126812) (end 140.295812 66.666) (width 0.1) (layer "F.Cu") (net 11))
 (segment (start 140.835 65.7775) (end 140.835 65.040001) (width 0.1) (layer "F.Cu") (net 11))
 (segment (start 139.386001 66.666) (end 139.235 66.514999) (width 0.1) (layer "F.Cu") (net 11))
 (segment (start 145 74.675) (end 145 71.705) (width 0.1) (layer "F.Cu") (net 11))
 (segment (start 140.835 65.7775) (end 140.835 66.126812) (width 0.1) (layer "F.Cu") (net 11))
 (segment (start 134.735001 71.14) (end 135.4725 71.14) (width 0.1) (layer "F.Cu") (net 19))
 (segment (start 143.7975 67.94) (end 143.11 67.94) (width 0.1) (layer "F.Cu") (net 31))
 (segment (start 143.7975 70.34) (end 144.146812 70.34) (width 0.1) (layer "F.Cu") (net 29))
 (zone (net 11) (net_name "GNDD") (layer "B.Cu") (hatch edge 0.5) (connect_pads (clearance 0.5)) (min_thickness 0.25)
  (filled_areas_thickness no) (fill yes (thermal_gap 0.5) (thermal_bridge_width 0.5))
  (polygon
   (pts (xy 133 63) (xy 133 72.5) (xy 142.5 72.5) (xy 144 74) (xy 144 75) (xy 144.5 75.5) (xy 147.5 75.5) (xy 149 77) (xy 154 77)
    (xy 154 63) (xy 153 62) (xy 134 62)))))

